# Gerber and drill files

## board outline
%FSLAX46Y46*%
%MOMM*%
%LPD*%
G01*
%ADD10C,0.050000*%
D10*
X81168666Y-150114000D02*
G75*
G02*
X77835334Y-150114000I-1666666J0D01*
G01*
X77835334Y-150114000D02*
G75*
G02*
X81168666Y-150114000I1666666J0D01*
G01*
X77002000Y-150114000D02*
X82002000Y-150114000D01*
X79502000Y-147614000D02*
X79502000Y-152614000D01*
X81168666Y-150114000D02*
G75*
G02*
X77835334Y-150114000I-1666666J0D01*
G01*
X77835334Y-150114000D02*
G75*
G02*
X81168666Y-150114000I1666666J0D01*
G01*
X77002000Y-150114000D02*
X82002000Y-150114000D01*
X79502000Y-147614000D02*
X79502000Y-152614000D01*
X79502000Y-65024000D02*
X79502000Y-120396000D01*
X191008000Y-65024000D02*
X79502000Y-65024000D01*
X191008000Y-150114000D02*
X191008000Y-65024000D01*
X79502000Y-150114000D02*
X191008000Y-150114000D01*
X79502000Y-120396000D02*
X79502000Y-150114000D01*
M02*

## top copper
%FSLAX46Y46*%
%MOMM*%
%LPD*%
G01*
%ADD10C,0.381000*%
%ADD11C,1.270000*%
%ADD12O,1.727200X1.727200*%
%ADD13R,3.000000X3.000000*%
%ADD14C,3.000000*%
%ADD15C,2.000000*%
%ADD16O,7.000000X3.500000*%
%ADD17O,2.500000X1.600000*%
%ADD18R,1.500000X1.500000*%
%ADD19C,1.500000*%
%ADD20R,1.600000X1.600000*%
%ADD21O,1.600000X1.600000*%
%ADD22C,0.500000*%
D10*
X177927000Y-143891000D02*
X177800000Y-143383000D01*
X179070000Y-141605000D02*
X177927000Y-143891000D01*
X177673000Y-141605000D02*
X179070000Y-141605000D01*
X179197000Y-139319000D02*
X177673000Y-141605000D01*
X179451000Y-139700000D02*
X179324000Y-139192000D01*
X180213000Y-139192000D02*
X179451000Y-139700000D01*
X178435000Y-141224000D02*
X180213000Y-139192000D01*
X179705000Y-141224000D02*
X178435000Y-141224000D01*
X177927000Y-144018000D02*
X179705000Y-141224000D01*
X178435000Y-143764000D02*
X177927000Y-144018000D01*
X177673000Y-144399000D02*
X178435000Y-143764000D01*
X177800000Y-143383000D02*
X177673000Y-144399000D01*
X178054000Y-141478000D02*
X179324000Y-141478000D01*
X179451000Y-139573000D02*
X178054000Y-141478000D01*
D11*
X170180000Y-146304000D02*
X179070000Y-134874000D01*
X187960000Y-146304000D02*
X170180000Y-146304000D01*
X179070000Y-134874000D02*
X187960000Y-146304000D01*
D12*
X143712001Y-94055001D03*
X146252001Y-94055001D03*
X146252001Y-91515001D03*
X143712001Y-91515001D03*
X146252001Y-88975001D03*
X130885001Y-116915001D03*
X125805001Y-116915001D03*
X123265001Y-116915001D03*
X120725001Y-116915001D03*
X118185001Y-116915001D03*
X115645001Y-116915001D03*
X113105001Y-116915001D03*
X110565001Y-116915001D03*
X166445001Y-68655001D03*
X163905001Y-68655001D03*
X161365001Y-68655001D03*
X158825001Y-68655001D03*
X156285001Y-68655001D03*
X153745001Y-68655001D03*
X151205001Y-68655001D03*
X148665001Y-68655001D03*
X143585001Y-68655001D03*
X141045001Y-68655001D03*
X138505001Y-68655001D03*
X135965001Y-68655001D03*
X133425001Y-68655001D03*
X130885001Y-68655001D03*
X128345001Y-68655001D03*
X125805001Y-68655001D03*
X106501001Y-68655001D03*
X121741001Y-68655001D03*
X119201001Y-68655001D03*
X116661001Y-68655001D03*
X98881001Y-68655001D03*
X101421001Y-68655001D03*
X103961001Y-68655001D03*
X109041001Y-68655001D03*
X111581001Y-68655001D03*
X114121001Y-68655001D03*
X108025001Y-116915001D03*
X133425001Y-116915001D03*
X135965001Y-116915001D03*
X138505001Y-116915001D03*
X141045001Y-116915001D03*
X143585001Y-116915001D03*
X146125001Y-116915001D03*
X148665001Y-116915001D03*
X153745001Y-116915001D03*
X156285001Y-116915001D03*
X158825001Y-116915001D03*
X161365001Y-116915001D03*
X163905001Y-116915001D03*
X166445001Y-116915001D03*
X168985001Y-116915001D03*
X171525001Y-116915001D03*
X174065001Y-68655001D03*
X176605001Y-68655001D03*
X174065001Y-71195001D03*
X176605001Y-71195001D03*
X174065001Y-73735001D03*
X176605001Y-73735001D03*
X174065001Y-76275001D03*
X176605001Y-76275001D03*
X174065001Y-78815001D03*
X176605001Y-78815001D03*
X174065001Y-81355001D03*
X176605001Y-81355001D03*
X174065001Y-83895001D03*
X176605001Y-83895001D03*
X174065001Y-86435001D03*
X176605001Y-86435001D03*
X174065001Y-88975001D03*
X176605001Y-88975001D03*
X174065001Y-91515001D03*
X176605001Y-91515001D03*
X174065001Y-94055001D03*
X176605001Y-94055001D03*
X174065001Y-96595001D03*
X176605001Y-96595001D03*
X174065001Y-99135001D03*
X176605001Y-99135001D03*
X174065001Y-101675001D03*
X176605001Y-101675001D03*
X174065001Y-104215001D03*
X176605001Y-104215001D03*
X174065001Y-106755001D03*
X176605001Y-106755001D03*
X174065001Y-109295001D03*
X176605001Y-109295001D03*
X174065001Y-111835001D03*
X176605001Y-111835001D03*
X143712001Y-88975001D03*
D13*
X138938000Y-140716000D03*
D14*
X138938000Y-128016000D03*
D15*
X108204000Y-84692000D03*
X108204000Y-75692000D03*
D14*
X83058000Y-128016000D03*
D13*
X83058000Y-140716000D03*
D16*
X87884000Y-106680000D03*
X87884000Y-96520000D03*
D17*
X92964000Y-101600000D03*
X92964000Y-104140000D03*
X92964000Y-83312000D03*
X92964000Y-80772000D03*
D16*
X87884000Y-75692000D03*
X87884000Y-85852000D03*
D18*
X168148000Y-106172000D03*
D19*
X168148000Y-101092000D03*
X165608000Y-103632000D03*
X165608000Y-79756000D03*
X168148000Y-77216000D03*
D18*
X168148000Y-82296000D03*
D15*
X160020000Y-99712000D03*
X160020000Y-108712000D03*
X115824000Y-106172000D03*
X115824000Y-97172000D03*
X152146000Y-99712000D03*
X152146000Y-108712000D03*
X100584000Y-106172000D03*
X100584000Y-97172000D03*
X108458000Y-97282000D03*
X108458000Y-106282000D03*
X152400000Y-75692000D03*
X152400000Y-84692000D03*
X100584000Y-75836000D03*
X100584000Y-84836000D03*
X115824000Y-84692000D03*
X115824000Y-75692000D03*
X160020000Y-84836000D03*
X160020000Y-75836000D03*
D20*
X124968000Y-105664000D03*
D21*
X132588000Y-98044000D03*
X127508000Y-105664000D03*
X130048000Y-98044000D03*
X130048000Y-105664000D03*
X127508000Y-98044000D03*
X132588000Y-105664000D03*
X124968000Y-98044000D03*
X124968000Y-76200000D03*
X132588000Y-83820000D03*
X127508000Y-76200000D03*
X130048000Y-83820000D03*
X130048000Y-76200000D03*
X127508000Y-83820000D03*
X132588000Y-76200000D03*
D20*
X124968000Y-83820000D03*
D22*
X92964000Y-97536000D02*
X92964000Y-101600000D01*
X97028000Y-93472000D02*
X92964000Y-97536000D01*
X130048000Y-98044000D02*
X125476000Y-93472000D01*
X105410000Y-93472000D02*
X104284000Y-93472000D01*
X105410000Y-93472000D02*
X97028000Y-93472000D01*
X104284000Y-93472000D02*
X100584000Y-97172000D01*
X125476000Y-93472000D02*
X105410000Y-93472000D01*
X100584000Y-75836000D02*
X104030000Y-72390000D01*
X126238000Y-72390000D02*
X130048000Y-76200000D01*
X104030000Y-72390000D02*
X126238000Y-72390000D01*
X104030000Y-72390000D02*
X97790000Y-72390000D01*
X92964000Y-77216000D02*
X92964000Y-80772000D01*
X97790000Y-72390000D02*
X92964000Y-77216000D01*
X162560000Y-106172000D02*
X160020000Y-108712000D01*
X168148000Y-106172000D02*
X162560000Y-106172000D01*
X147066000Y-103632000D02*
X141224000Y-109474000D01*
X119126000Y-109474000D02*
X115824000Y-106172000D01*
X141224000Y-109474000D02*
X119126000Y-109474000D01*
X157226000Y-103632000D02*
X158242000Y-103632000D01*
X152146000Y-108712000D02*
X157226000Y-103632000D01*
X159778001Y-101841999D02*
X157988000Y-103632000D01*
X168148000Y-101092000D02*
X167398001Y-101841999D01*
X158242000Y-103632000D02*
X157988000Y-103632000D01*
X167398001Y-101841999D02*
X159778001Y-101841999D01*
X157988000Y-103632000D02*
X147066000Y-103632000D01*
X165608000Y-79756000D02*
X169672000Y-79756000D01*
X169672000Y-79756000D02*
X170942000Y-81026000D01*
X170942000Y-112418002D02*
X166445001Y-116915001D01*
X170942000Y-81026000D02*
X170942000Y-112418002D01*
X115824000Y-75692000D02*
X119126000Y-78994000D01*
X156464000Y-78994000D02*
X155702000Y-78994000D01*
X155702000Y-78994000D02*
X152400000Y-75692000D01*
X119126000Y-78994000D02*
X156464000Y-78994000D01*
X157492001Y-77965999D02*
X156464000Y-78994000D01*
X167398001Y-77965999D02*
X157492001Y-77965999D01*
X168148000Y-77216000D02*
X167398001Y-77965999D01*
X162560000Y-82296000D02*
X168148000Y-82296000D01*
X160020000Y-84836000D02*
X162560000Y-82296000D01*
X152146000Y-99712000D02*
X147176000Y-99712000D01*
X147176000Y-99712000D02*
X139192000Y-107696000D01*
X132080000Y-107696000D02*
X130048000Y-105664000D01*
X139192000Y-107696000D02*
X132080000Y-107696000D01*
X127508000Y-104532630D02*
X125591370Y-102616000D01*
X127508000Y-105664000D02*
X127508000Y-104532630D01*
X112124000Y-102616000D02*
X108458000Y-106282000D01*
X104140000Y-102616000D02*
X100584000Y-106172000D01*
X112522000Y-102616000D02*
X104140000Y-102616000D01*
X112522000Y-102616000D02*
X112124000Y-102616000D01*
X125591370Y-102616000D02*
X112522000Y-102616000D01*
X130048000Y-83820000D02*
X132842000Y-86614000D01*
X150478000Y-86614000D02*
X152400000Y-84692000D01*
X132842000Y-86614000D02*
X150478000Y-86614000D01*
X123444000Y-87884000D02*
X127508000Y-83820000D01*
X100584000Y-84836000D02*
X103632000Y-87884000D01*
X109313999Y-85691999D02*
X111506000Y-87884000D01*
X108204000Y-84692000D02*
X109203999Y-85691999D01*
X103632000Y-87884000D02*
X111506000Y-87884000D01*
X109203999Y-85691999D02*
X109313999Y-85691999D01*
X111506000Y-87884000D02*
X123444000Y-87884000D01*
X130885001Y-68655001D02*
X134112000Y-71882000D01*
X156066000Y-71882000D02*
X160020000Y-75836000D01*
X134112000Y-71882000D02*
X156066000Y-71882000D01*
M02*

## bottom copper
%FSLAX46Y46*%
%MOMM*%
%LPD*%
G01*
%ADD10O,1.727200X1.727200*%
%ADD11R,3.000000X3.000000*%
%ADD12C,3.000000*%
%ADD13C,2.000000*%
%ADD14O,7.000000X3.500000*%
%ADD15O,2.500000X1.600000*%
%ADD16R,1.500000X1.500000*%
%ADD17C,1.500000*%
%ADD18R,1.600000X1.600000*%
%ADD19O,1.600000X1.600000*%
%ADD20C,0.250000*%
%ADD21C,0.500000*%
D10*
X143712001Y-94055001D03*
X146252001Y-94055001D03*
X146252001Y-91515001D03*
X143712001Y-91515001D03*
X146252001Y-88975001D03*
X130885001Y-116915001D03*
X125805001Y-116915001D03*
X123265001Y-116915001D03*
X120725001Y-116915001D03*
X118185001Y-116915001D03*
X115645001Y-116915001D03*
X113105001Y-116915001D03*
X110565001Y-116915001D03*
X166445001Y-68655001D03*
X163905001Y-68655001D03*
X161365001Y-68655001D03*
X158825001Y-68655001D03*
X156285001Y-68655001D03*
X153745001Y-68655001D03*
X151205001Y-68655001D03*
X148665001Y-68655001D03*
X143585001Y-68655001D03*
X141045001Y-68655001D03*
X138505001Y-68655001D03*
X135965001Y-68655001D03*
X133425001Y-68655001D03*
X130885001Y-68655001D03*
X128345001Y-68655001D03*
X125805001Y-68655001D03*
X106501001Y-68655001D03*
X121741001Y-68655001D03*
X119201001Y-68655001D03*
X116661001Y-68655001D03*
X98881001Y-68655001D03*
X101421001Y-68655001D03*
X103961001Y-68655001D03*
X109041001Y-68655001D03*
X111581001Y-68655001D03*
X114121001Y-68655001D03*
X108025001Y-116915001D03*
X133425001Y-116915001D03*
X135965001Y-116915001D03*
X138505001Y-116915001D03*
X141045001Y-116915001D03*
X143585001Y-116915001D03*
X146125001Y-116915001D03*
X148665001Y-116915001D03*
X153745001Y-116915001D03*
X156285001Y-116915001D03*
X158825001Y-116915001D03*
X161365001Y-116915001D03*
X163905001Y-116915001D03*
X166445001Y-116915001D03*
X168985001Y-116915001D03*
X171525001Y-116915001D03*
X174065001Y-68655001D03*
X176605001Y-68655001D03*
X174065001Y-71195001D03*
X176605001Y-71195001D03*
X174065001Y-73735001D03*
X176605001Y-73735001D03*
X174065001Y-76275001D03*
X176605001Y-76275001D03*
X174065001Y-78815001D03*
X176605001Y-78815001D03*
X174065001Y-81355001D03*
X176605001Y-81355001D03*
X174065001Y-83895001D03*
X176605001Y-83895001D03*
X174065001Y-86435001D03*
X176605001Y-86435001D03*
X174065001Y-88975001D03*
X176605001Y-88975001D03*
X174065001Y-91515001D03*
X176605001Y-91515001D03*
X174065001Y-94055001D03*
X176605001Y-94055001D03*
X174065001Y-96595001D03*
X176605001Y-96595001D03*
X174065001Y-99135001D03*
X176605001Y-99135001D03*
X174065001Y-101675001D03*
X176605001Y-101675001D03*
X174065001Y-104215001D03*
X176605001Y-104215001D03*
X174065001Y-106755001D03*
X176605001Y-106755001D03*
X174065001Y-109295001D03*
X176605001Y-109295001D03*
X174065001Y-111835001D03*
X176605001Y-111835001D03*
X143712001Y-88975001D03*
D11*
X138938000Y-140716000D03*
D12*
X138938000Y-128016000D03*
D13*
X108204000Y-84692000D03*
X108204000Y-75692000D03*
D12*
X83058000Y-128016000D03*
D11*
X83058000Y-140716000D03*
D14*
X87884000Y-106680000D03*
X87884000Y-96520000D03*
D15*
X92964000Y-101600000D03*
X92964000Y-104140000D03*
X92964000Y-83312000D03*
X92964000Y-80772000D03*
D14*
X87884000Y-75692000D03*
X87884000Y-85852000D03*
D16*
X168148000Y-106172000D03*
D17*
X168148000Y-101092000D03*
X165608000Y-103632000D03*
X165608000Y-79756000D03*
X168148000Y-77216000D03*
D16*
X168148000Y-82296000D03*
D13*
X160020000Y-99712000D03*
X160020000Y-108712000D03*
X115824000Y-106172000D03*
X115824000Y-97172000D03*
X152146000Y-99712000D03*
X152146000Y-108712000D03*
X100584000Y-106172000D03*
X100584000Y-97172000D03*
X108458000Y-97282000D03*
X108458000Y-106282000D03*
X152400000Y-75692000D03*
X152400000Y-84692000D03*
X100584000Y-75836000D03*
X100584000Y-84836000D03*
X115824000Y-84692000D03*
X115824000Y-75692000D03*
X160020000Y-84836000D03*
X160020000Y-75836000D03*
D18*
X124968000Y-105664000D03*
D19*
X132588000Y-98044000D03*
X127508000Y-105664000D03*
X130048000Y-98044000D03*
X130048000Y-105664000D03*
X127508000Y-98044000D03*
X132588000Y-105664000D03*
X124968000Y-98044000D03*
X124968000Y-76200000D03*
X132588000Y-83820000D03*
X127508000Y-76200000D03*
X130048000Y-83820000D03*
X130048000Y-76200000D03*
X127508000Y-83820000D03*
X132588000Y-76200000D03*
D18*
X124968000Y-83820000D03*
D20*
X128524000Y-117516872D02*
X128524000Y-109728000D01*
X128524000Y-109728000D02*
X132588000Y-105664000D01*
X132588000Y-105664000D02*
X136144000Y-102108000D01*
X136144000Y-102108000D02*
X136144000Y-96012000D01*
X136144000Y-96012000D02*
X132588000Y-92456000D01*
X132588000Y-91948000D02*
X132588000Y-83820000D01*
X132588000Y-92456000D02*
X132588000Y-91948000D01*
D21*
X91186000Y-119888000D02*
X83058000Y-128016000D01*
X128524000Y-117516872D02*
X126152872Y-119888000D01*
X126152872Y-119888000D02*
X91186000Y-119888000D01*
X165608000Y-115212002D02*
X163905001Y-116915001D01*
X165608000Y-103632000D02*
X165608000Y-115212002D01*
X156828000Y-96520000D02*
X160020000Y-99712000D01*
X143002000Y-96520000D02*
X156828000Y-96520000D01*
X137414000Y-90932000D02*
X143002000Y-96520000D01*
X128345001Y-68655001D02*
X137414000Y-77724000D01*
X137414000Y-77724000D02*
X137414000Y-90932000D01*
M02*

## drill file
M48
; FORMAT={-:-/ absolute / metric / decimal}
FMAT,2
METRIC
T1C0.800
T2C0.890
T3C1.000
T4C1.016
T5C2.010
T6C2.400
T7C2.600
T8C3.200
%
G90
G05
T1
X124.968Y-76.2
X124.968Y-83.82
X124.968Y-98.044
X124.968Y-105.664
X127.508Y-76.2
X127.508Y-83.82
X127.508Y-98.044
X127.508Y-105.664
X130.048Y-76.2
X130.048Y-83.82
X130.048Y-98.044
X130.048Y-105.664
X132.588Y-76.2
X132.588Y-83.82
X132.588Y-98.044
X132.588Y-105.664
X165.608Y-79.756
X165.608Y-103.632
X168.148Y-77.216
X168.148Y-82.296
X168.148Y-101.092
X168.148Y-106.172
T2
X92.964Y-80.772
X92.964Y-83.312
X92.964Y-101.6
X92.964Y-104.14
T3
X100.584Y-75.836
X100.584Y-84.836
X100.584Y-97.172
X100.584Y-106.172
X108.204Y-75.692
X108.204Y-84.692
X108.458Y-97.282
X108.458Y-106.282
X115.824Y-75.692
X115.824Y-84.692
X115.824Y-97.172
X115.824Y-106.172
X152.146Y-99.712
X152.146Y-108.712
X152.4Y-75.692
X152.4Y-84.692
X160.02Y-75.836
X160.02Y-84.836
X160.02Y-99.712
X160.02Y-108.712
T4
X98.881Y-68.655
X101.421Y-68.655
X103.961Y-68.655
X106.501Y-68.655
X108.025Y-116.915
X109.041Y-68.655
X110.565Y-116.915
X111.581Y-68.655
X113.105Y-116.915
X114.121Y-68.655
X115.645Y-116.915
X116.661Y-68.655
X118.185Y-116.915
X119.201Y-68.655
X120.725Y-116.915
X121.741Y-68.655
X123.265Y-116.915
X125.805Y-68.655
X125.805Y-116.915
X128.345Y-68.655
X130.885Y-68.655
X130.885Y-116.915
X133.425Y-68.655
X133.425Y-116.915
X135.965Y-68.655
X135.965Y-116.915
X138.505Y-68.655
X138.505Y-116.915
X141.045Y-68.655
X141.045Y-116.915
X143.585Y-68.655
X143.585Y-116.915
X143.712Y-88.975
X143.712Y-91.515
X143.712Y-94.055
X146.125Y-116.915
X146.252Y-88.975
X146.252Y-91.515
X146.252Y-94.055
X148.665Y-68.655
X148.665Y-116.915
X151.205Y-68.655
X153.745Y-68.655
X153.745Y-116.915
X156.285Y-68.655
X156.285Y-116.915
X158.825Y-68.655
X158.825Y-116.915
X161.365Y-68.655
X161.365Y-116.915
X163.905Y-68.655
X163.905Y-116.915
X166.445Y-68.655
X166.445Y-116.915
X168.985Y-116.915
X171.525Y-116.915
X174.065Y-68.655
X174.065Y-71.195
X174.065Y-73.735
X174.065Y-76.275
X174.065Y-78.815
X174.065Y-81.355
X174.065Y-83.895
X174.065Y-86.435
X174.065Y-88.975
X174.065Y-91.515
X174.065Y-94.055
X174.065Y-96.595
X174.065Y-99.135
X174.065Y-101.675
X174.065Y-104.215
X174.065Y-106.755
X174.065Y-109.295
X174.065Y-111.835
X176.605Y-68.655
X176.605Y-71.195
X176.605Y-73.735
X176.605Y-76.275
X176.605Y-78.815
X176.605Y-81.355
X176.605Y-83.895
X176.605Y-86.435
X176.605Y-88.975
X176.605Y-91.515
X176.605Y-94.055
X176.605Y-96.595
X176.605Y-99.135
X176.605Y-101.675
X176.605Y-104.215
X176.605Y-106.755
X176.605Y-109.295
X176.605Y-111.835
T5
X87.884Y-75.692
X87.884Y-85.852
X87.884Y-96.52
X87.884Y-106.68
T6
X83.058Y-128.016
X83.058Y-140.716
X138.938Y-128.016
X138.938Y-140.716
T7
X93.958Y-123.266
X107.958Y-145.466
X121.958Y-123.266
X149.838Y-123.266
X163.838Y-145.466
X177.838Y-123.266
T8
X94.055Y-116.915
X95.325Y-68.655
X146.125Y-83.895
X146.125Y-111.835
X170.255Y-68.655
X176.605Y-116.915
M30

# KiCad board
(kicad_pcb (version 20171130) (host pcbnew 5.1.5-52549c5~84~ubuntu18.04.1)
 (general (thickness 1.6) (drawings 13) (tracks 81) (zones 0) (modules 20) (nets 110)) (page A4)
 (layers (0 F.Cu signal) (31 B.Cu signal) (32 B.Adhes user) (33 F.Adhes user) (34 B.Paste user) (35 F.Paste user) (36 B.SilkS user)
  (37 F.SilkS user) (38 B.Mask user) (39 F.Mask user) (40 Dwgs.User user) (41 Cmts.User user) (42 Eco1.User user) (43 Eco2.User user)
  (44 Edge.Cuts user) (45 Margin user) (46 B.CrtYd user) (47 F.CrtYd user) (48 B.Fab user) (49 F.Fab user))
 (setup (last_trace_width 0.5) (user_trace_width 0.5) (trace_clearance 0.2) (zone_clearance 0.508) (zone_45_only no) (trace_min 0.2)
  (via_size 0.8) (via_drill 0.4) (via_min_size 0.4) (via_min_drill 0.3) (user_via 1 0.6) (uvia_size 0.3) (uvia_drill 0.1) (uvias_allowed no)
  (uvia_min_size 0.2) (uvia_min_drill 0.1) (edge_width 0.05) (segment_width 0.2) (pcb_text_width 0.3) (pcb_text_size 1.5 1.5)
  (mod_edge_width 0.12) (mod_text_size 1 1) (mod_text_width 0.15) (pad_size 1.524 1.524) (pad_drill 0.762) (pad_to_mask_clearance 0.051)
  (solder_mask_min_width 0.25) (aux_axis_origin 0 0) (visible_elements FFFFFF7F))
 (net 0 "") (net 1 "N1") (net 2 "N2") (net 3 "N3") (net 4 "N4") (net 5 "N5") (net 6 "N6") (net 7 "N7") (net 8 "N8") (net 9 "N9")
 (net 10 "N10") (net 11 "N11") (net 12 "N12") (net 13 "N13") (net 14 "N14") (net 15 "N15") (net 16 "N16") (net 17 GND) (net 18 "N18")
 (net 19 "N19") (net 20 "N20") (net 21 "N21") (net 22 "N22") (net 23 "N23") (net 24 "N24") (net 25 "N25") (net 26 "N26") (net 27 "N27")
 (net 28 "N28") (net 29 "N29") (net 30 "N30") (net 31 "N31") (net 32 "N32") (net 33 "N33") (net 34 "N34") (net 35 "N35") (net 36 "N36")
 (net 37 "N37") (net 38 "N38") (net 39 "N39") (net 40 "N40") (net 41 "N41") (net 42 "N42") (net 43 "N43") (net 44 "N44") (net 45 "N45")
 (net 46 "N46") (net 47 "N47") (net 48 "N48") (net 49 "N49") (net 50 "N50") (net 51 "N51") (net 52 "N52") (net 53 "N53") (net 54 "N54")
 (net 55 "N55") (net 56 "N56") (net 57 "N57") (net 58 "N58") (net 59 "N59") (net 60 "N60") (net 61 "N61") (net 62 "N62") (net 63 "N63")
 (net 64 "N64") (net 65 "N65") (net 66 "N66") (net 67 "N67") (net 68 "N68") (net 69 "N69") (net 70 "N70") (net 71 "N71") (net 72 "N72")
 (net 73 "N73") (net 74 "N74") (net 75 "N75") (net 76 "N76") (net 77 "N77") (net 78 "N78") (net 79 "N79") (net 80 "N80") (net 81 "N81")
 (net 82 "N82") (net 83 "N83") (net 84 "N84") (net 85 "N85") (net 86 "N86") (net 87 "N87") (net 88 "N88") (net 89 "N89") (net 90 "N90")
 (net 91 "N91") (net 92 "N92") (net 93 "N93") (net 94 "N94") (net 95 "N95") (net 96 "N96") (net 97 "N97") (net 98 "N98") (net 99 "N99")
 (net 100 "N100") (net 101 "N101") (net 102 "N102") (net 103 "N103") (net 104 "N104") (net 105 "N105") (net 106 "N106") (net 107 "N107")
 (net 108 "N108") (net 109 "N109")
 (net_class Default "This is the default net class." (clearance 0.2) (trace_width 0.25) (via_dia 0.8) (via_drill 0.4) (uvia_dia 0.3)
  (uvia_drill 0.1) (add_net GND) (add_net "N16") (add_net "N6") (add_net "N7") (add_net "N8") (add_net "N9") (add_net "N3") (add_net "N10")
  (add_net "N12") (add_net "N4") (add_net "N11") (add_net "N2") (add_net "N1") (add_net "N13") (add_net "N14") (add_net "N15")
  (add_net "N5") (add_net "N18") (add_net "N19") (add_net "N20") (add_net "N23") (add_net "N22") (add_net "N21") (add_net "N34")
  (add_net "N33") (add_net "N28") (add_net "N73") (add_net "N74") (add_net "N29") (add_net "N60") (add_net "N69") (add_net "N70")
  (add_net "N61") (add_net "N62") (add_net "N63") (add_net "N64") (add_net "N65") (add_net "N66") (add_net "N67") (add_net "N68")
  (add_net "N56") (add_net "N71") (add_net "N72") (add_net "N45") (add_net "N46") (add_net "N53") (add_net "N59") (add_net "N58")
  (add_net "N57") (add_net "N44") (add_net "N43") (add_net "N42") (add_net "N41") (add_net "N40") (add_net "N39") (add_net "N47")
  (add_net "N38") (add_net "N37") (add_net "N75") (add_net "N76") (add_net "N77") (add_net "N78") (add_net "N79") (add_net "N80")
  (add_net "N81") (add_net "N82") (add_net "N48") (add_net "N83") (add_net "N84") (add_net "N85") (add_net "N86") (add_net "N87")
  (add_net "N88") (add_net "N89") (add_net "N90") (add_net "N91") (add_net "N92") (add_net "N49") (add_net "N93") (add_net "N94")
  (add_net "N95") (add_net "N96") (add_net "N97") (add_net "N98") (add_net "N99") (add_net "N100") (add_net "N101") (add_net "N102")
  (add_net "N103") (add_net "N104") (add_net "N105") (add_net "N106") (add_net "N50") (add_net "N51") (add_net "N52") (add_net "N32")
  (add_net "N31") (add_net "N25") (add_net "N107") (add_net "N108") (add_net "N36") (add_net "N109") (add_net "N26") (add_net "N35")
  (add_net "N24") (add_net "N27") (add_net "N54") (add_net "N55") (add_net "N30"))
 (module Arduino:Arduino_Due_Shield (layer F.Cu) (at 80.085001 119.455001)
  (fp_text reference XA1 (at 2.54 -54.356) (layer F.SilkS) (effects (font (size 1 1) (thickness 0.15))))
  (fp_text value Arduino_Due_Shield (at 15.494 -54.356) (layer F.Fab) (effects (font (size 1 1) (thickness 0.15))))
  (pad RST2 thru_hole oval (at 63.627 -25.4) (size 1.7272 1.7272) (drill 1.016) (layers *.Cu *.Mask))
  (pad GND4 thru_hole oval (at 66.167 -25.4) (size 1.7272 1.7272) (drill 1.016) (layers *.Cu *.Mask))
  (pad MOSI thru_hole oval (at 66.167 -27.94) (size 1.7272 1.7272) (drill 1.016) (layers *.Cu *.Mask))
  (pad SCK thru_hole oval (at 63.627 -27.94) (size 1.7272 1.7272) (drill 1.016) (layers *.Cu *.Mask))
  (pad 5V2 thru_hole oval (at 66.167 -30.48) (size 1.7272 1.7272) (drill 1.016) (layers *.Cu *.Mask))
  (pad A0 thru_hole oval (at 50.8 -2.54) (size 1.7272 1.7272) (drill 1.016) (layers *.Cu *.Mask))
  (pad VIN thru_hole oval (at 45.72 -2.54) (size 1.7272 1.7272) (drill 1.016) (layers *.Cu *.Mask))
  (pad GND3 thru_hole oval (at 43.18 -2.54) (size 1.7272 1.7272) (drill 1.016) (layers *.Cu *.Mask))
  (pad GND2 thru_hole oval (at 40.64 -2.54) (size 1.7272 1.7272) (drill 1.016) (layers *.Cu *.Mask))
  (pad 5V1 thru_hole oval (at 38.1 -2.54) (size 1.7272 1.7272) (drill 1.016) (layers *.Cu *.Mask))
  (pad 3V3 thru_hole oval (at 35.56 -2.54) (size 1.7272 1.7272) (drill 1.016) (layers *.Cu *.Mask))
  (pad RST1 thru_hole oval (at 33.02 -2.54) (size 1.7272 1.7272) (drill 1.016) (layers *.Cu *.Mask))
  (pad IORF thru_hole oval (at 30.48 -2.54) (size 1.7272 1.7272) (drill 1.016) (layers *.Cu *.Mask))
  (pad D21 thru_hole oval (at 86.36 -50.8) (size 1.7272 1.7272) (drill 1.016) (layers *.Cu *.Mask))
  (pad D20 thru_hole oval (at 83.82 -50.8) (size 1.7272 1.7272) (drill 1.016) (layers *.Cu *.Mask))
  (pad D19 thru_hole oval (at 81.28 -50.8) (size 1.7272 1.7272) (drill 1.016) (layers *.Cu *.Mask))
  (pad D18 thru_hole oval (at 78.74 -50.8) (size 1.7272 1.7272) (drill 1.016) (layers *.Cu *.Mask))
  (pad D17 thru_hole oval (at 76.2 -50.8) (size 1.7272 1.7272) (drill 1.016) (layers *.Cu *.Mask))
  (pad D16 thru_hole oval (at 73.66 -50.8) (size 1.7272 1.7272) (drill 1.016) (layers *.Cu *.Mask))
  (pad D15 thru_hole oval (at 71.12 -50.8) (size 1.7272 1.7272) (drill 1.016) (layers *.Cu *.Mask))
  (pad D14 thru_hole oval (at 68.58 -50.8) (size 1.7272 1.7272) (drill 1.016) (layers *.Cu *.Mask))
  (pad D0 thru_hole oval (at 63.5 -50.8) (size 1.7272 1.7272) (drill 1.016) (layers *.Cu *.Mask))
  (pad D1 thru_hole oval (at 60.96 -50.8) (size 1.7272 1.7272) (drill 1.016) (layers *.Cu *.Mask))
  (pad D2 thru_hole oval (at 58.42 -50.8) (size 1.7272 1.7272) (drill 1.016) (layers *.Cu *.Mask))
  (pad D3 thru_hole oval (at 55.88 -50.8) (size 1.7272 1.7272) (drill 1.016) (layers *.Cu *.Mask))
  (pad D4 thru_hole oval (at 53.34 -50.8) (size 1.7272 1.7272) (drill 1.016) (layers *.Cu *.Mask))
  (pad D5 thru_hole oval (at 50.8 -50.8) (size 1.7272 1.7272) (drill 1.016) (layers *.Cu *.Mask) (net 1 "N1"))
  (pad D6 thru_hole oval (at 48.26 -50.8) (size 1.7272 1.7272) (drill 1.016) (layers *.Cu *.Mask) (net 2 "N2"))
  (pad D7 thru_hole oval (at 45.72 -50.8) (size 1.7272 1.7272) (drill 1.016) (layers *.Cu *.Mask))
  (pad GND1 thru_hole oval (at 26.416 -50.8) (size 1.7272 1.7272) (drill 1.016) (layers *.Cu *.Mask))
  (pad D8 thru_hole oval (at 41.656 -50.8) (size 1.7272 1.7272) (drill 1.016) (layers *.Cu *.Mask))
  (pad D9 thru_hole oval (at 39.116 -50.8) (size 1.7272 1.7272) (drill 1.016) (layers *.Cu *.Mask))
  (pad D10 thru_hole oval (at 36.576 -50.8) (size 1.7272 1.7272) (drill 1.016) (layers *.Cu *.Mask))
  (pad "" np_thru_hole circle (at 66.04 -7.62) (size 3.2 3.2) (drill 3.2) (layers *.Cu *.Mask))
  (pad "" np_thru_hole circle (at 66.04 -35.56) (size 3.2 3.2) (drill 3.2) (layers *.Cu *.Mask))
  (pad "" np_thru_hole circle (at 90.17 -50.8) (size 3.2 3.2) (drill 3.2) (layers *.Cu *.Mask))
  (pad "" np_thru_hole circle (at 15.24 -50.8) (size 3.2 3.2) (drill 3.2) (layers *.Cu *.Mask))
  (pad "" np_thru_hole circle (at 96.52 -2.54) (size 3.2 3.2) (drill 3.2) (layers *.Cu *.Mask))
  (pad "" np_thru_hole circle (at 13.97 -2.54) (size 3.2 3.2) (drill 3.2) (layers *.Cu *.Mask))
  (pad SCL1 thru_hole oval (at 18.796 -50.8) (size 1.7272 1.7272) (drill 1.016) (layers *.Cu *.Mask))
  (pad SDA1 thru_hole oval (at 21.336 -50.8) (size 1.7272 1.7272) (drill 1.016) (layers *.Cu *.Mask))
  (pad AREF thru_hole oval (at 23.876 -50.8) (size 1.7272 1.7272) (drill 1.016) (layers *.Cu *.Mask))
  (pad D13 thru_hole oval (at 28.956 -50.8) (size 1.7272 1.7272) (drill 1.016) (layers *.Cu *.Mask))
  (pad D12 thru_hole oval (at 31.496 -50.8) (size 1.7272 1.7272) (drill 1.016) (layers *.Cu *.Mask))
  (pad D11 thru_hole oval (at 34.036 -50.8) (size 1.7272 1.7272) (drill 1.016) (layers *.Cu *.Mask))
  (pad "" thru_hole oval (at 27.94 -2.54) (size 1.7272 1.7272) (drill 1.016) (layers *.Cu *.Mask))
  (pad A1 thru_hole oval (at 53.34 -2.54) (size 1.7272 1.7272) (drill 1.016) (layers *.Cu *.Mask))
  (pad A2 thru_hole oval (at 55.88 -2.54) (size 1.7272 1.7272) (drill 1.016) (layers *.Cu *.Mask))
  (pad A3 thru_hole oval (at 58.42 -2.54) (size 1.7272 1.7272) (drill 1.016) (layers *.Cu *.Mask))
  (pad A4 thru_hole oval (at 60.96 -2.54) (size 1.7272 1.7272) (drill 1.016) (layers *.Cu *.Mask))
  (pad A5 thru_hole oval (at 63.5 -2.54) (size 1.7272 1.7272) (drill 1.016) (layers *.Cu *.Mask))
  (pad A6 thru_hole oval (at 66.04 -2.54) (size 1.7272 1.7272) (drill 1.016) (layers *.Cu *.Mask))
  (pad A7 thru_hole oval (at 68.58 -2.54) (size 1.7272 1.7272) (drill 1.016) (layers *.Cu *.Mask))
  (pad A8 thru_hole oval (at 73.66 -2.54) (size 1.7272 1.7272) (drill 1.016) (layers *.Cu *.Mask))
  (pad A9 thru_hole oval (at 76.2 -2.54) (size 1.7272 1.7272) (drill 1.016) (layers *.Cu *.Mask))
  (pad A10 thru_hole oval (at 78.74 -2.54) (size 1.7272 1.7272) (drill 1.016) (layers *.Cu *.Mask))
  (pad A11 thru_hole oval (at 81.28 -2.54) (size 1.7272 1.7272) (drill 1.016) (layers *.Cu *.Mask))
  (pad DAC0 thru_hole oval (at 83.82 -2.54) (size 1.7272 1.7272) (drill 1.016) (layers *.Cu *.Mask) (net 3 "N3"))
  (pad DAC1 thru_hole oval (at 86.36 -2.54) (size 1.7272 1.7272) (drill 1.016) (layers *.Cu *.Mask) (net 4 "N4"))
  (pad CANR thru_hole oval (at 88.9 -2.54) (size 1.7272 1.7272) (drill 1.016) (layers *.Cu *.Mask))
  (pad CANT thru_hole oval (at 91.44 -2.54) (size 1.7272 1.7272) (drill 1.016) (layers *.Cu *.Mask))
  (pad 5V3 thru_hole oval (at 93.98 -50.8) (size 1.7272 1.7272) (drill 1.016) (layers *.Cu *.Mask))
  (pad 5V4 thru_hole oval (at 96.52 -50.8) (size 1.7272 1.7272) (drill 1.016) (layers *.Cu *.Mask))
  (pad D22 thru_hole oval (at 93.98 -48.26) (size 1.7272 1.7272) (drill 1.016) (layers *.Cu *.Mask))
  (pad D23 thru_hole oval (at 96.52 -48.26) (size 1.7272 1.7272) (drill 1.016) (layers *.Cu *.Mask))
  (pad D24 thru_hole oval (at 93.98 -45.72) (size 1.7272 1.7272) (drill 1.016) (layers *.Cu *.Mask))
  (pad D25 thru_hole oval (at 96.52 -45.72) (size 1.7272 1.7272) (drill 1.016) (layers *.Cu *.Mask))
  (pad D26 thru_hole oval (at 93.98 -43.18) (size 1.7272 1.7272) (drill 1.016) (layers *.Cu *.Mask))
  (pad D27 thru_hole oval (at 96.52 -43.18) (size 1.7272 1.7272) (drill 1.016) (layers *.Cu *.Mask))
  (pad D28 thru_hole oval (at 93.98 -40.64) (size 1.7272 1.7272) (drill 1.016) (layers *.Cu *.Mask))
  (pad D29 thru_hole oval (at 96.52 -40.64) (size 1.7272 1.7272) (drill 1.016) (layers *.Cu *.Mask))
  (pad D30 thru_hole oval (at 93.98 -38.1) (size 1.7272 1.7272) (drill 1.016) (layers *.Cu *.Mask))
  (pad D31 thru_hole oval (at 96.52 -38.1) (size 1.7272 1.7272) (drill 1.016) (layers *.Cu *.Mask))
  (pad D32 thru_hole oval (at 93.98 -35.56) (size 1.7272 1.7272) (drill 1.016) (layers *.Cu *.Mask))
  (pad D33 thru_hole oval (at 96.52 -35.56) (size 1.7272 1.7272) (drill 1.016) (layers *.Cu *.Mask))
  (pad D34 thru_hole oval (at 93.98 -33.02) (size 1.7272 1.7272) (drill 1.016) (layers *.Cu *.Mask))
  (pad D35 thru_hole oval (at 96.52 -33.02) (size 1.7272 1.7272) (drill 1.016) (layers *.Cu *.Mask))
  (pad D36 thru_hole oval (at 93.98 -30.48) (size 1.7272 1.7272) (drill 1.016) (layers *.Cu *.Mask))
  (pad D37 thru_hole oval (at 96.52 -30.48) (size 1.7272 1.7272) (drill 1.016) (layers *.Cu *.Mask))
  (pad D38 thru_hole oval (at 93.98 -27.94) (size 1.7272 1.7272) (drill 1.016) (layers *.Cu *.Mask))
  (pad D39 thru_hole oval (at 96.52 -27.94) (size 1.7272 1.7272) (drill 1.016) (layers *.Cu *.Mask))
  (pad D40 thru_hole oval (at 93.98 -25.4) (size 1.7272 1.7272) (drill 1.016) (layers *.Cu *.Mask))
  (pad D41 thru_hole oval (at 96.52 -25.4) (size 1.7272 1.7272) (drill 1.016) (layers *.Cu *.Mask))
  (pad D42 thru_hole oval (at 93.98 -22.86) (size 1.7272 1.7272) (drill 1.016) (layers *.Cu *.Mask))
  (pad D43 thru_hole oval (at 96.52 -22.86) (size 1.7272 1.7272) (drill 1.016) (layers *.Cu *.Mask))
  (pad D44 thru_hole oval (at 93.98 -20.32) (size 1.7272 1.7272) (drill 1.016) (layers *.Cu *.Mask))
  (pad D45 thru_hole oval (at 96.52 -20.32) (size 1.7272 1.7272) (drill 1.016) (layers *.Cu *.Mask))
  (pad D46 thru_hole oval (at 93.98 -17.78) (size 1.7272 1.7272) (drill 1.016) (layers *.Cu *.Mask))
  (pad D47 thru_hole oval (at 96.52 -17.78) (size 1.7272 1.7272) (drill 1.016) (layers *.Cu *.Mask))
  (pad D48 thru_hole oval (at 93.98 -15.24) (size 1.7272 1.7272) (drill 1.016) (layers *.Cu *.Mask))
  (pad D49 thru_hole oval (at 96.52 -15.24) (size 1.7272 1.7272) (drill 1.016) (layers *.Cu *.Mask))
  (pad D50 thru_hole oval (at 93.98 -12.7) (size 1.7272 1.7272) (drill 1.016) (layers *.Cu *.Mask))
  (pad D51 thru_hole oval (at 96.52 -12.7) (size 1.7272 1.7272) (drill 1.016) (layers *.Cu *.Mask))
  (pad D52 thru_hole oval (at 93.98 -10.16) (size 1.7272 1.7272) (drill 1.016) (layers *.Cu *.Mask))
  (pad D53 thru_hole oval (at 96.52 -10.16) (size 1.7272 1.7272) (drill 1.016) (layers *.Cu *.Mask))
  (pad GND5 thru_hole oval (at 93.98 -7.62) (size 1.7272 1.7272) (drill 1.016) (layers *.Cu *.Mask))
  (pad GND6 thru_hole oval (at 96.52 -7.62) (size 1.7272 1.7272) (drill 1.016) (layers *.Cu *.Mask))
  (pad MISO thru_hole oval (at 63.627 -30.48) (size 1.7272 1.7272) (drill 1.016) (layers *.Cu *.Mask)))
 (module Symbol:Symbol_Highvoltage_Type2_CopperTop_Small (layer F.Cu) (at 179.07 142.494)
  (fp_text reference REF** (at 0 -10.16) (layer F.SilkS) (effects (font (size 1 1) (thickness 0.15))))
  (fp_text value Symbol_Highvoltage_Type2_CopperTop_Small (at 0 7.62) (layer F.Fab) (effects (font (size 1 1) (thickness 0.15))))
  (fp_line (start -1.143 1.397) (end -1.27 0.889) (layer F.Cu) (width 0.381))
  (fp_line (start 0 -0.889) (end -1.143 1.397) (layer F.Cu) (width 0.381))
  (fp_line (start -1.397 -0.889) (end 0 -0.889) (layer F.Cu) (width 0.381))
  (fp_line (start 0.127 -3.175) (end -1.397 -0.889) (layer F.Cu) (width 0.381))
  (fp_line (start 0.381 -2.794) (end 0.254 -3.302) (layer F.Cu) (width 0.381))
  (fp_line (start 1.143 -3.302) (end 0.381 -2.794) (layer F.Cu) (width 0.381))
  (fp_line (start -0.635 -1.27) (end 1.143 -3.302) (layer F.Cu) (width 0.381))
  (fp_line (start 0.635 -1.27) (end -0.635 -1.27) (layer F.Cu) (width 0.381))
  (fp_line (start -1.143 1.524) (end 0.635 -1.27) (layer F.Cu) (width 0.381))
  (fp_line (start -0.635 1.27) (end -1.143 1.524) (layer F.Cu) (width 0.381))
  (fp_line (start -1.397 1.905) (end -0.635 1.27) (layer F.Cu) (width 0.381))
  (fp_line (start -1.27 0.889) (end -1.397 1.905) (layer F.Cu) (width 0.381))
  (fp_line (start -1.016 -1.016) (end 0.254 -1.016) (layer F.Cu) (width 0.381))
  (fp_line (start 0.381 -2.921) (end -1.016 -1.016) (layer F.Cu) (width 0.381))
  (fp_line (start -8.89 3.81) (end 0 -7.62) (layer F.Cu) (width 1.27))
  (fp_line (start 8.89 3.81) (end -8.89 3.81) (layer F.Cu) (width 1.27))
  (fp_line (start 0 -7.62) (end 8.89 3.81) (layer F.Cu) (width 1.27)))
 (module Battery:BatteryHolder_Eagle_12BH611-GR (layer B.Cu) (at 138.938 140.716 180)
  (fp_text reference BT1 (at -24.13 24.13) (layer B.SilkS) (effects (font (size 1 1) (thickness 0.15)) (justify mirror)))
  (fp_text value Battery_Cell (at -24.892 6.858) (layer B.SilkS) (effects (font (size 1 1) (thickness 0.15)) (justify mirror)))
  (pad "" np_thru_hole circle (at -24.9 -4.75 180) (size 2.6 2.6) (drill 2.6) (layers *.Cu *.Mask))
  (pad "" np_thru_hole circle (at -38.9 17.45 180) (size 2.6 2.6) (drill 2.6) (layers *.Cu *.Mask))
  (pad "" np_thru_hole circle (at -10.9 17.45 180) (size 2.6 2.6) (drill 2.6) (layers *.Cu *.Mask))
  (pad 1 thru_hole rect (at 0 0 180) (size 3 3) (drill 2.4) (layers *.Cu *.Mask))
  (pad 2 thru_hole circle (at 0 12.7 180) (size 3 3) (drill 2.4) (layers *.Cu *.Mask)))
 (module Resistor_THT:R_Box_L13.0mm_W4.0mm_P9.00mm (layer F.Cu) (at 108.204 75.692 270)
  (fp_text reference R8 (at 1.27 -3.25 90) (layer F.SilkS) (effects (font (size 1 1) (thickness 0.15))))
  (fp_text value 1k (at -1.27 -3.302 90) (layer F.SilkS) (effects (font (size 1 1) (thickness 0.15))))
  (pad 2 thru_hole circle (at 9 0 270) (size 2 2) (drill 1) (layers *.Cu *.Mask) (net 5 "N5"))
  (pad 1 thru_hole circle (at 0 0 270) (size 2 2) (drill 1) (layers *.Cu *.Mask)))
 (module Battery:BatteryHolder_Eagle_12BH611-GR (layer B.Cu) (at 83.058 140.716 180)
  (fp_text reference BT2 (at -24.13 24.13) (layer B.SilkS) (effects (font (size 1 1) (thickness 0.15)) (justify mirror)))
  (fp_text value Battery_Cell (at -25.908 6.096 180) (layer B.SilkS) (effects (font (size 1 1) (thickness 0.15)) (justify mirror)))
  (pad 2 thru_hole circle (at 0 12.7 180) (size 3 3) (drill 2.4) (layers *.Cu *.Mask) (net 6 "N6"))
  (pad 1 thru_hole rect (at 0 0 180) (size 3 3) (drill 2.4) (layers *.Cu *.Mask))
  (pad "" np_thru_hole circle (at -10.9 17.45 180) (size 2.6 2.6) (drill 2.6) (layers *.Cu *.Mask))
  (pad "" np_thru_hole circle (at -38.9 17.45 180) (size 2.6 2.6) (drill 2.6) (layers *.Cu *.Mask))
  (pad "" np_thru_hole circle (at -24.9 -4.75 180) (size 2.6 2.6) (drill 2.6) (layers *.Cu *.Mask)))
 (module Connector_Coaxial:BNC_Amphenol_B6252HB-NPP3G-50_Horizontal (layer F.Cu) (at 92.964 101.6 90)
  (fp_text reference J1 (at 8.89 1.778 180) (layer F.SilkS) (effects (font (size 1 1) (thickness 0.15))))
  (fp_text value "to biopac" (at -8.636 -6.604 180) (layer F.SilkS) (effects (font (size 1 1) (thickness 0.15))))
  (pad 2 thru_hole oval (at -5.08 -5.08 90) (size 3.5 7) (drill 2.01) (layers *.Cu *.Mask))
  (pad 2 thru_hole oval (at 5.08 -5.08 90) (size 3.5 7) (drill 2.01) (layers *.Cu *.Mask))
  (pad 1 thru_hole oval (at 0 0 90) (size 1.6 2.5) (drill 0.89) (layers *.Cu *.Mask) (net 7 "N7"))
  (pad 2 thru_hole oval (at -2.54 0 90) (size 1.6 2.5) (drill 0.89) (layers *.Cu *.Mask)))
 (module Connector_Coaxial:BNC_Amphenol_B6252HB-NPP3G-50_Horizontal (layer F.Cu) (at 92.964 80.772 90)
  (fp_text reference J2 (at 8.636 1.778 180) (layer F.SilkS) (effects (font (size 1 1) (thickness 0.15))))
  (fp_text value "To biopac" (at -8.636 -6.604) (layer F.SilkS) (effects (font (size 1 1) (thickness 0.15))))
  (pad 2 thru_hole oval (at -2.54 0 90) (size 1.6 2.5) (drill 0.89) (layers *.Cu *.Mask))
  (pad 1 thru_hole oval (at 0 0 90) (size 1.6 2.5) (drill 0.89) (layers *.Cu *.Mask) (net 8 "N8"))
  (pad 2 thru_hole oval (at 5.08 -5.08 90) (size 3.5 7) (drill 2.01) (layers *.Cu *.Mask))
  (pad 2 thru_hole oval (at -5.08 -5.08 90) (size 3.5 7) (drill 2.01) (layers *.Cu *.Mask)))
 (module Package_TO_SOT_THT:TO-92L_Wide (layer F.Cu) (at 168.148 106.172 90)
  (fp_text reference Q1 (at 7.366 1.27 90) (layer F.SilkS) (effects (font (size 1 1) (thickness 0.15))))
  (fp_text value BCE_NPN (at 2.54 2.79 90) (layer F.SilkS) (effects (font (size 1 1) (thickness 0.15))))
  (pad 1 thru_hole rect (at 0 0 180) (size 1.5 1.5) (drill 0.8) (layers *.Cu *.Mask) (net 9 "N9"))
  (pad 3 thru_hole circle (at 5.08 0 180) (size 1.5 1.5) (drill 0.8) (layers *.Cu *.Mask) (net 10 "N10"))
  (pad 2 thru_hole circle (at 2.54 -2.54 180) (size 1.5 1.5) (drill 0.8) (layers *.Cu *.Mask) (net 3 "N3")))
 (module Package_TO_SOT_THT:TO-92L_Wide (layer F.Cu) (at 168.148 82.296 90)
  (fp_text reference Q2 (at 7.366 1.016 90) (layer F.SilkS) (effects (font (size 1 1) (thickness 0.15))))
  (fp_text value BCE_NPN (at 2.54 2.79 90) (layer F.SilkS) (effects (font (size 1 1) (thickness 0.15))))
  (pad 2 thru_hole circle (at 2.54 -2.54 180) (size 1.5 1.5) (drill 0.8) (layers *.Cu *.Mask) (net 4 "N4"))
  (pad 3 thru_hole circle (at 5.08 0 180) (size 1.5 1.5) (drill 0.8) (layers *.Cu *.Mask) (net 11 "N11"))
  (pad 1 thru_hole rect (at 0 0 180) (size 1.5 1.5) (drill 0.8) (layers *.Cu *.Mask) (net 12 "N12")))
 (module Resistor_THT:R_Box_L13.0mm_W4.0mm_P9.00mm (layer F.Cu) (at 160.02 108.712 90)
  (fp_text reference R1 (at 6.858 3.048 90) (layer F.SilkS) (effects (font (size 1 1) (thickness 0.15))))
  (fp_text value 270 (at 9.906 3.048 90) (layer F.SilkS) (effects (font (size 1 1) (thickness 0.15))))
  (pad 2 thru_hole circle (at 9 0 90) (size 2 2) (drill 1) (layers *.Cu *.Mask) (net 2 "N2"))
  (pad 1 thru_hole circle (at 0 0 90) (size 2 2) (drill 1) (layers *.Cu *.Mask) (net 9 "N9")))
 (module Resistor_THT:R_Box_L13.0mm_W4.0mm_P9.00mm (layer F.Cu) (at 115.824 106.172 90)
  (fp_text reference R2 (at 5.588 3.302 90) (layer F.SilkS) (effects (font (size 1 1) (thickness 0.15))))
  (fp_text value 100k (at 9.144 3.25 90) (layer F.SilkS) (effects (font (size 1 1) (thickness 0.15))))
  (pad 1 thru_hole circle (at 0 0 90) (size 2 2) (drill 1) (layers *.Cu *.Mask) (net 10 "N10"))
  (pad 2 thru_hole circle (at 9 0 90) (size 2 2) (drill 1) (layers *.Cu *.Mask)))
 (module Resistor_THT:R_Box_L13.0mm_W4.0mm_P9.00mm (layer F.Cu) (at 152.146 108.712 90)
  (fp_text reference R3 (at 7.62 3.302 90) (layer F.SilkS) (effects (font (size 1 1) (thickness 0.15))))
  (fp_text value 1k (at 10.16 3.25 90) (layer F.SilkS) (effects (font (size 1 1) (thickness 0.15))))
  (pad 2 thru_hole circle (at 9 0 90) (size 2 2) (drill 1) (layers *.Cu *.Mask) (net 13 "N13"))
  (pad 1 thru_hole circle (at 0 0 90) (size 2 2) (drill 1) (layers *.Cu *.Mask) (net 10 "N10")))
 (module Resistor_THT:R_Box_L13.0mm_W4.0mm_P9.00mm (layer F.Cu) (at 100.584 106.172 90)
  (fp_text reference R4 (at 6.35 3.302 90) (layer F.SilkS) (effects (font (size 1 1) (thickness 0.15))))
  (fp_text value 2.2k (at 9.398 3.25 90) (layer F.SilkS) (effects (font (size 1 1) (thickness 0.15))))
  (pad 1 thru_hole circle (at 0 0 90) (size 2 2) (drill 1) (layers *.Cu *.Mask) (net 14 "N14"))
  (pad 2 thru_hole circle (at 9 0 90) (size 2 2) (drill 1) (layers *.Cu *.Mask) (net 7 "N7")))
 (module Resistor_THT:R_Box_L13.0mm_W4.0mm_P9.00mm (layer F.Cu) (at 108.458 97.282 270)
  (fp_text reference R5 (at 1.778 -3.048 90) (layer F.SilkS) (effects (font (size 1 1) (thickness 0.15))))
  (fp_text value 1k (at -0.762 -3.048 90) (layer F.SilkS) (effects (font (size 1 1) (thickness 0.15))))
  (pad 1 thru_hole circle (at 0 0 270) (size 2 2) (drill 1) (layers *.Cu *.Mask))
  (pad 2 thru_hole circle (at 9 0 270) (size 2 2) (drill 1) (layers *.Cu *.Mask) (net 14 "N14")))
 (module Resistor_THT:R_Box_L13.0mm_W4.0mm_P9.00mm (layer F.Cu) (at 152.4 75.692 270)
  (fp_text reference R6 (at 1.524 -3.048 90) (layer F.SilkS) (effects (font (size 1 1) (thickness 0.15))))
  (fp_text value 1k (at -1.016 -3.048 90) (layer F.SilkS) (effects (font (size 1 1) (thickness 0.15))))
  (pad 1 thru_hole circle (at 0 0 270) (size 2 2) (drill 1) (layers *.Cu *.Mask) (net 11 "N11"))
  (pad 2 thru_hole circle (at 9 0 270) (size 2 2) (drill 1) (layers *.Cu *.Mask) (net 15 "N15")))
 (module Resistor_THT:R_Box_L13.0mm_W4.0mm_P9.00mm (layer F.Cu) (at 100.584 84.836 90)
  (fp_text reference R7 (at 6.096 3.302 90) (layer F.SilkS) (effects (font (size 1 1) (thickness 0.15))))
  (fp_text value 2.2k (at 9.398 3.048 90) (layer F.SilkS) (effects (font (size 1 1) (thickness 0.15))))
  (pad 2 thru_hole circle (at 9 0 90) (size 2 2) (drill 1) (layers *.Cu *.Mask) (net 8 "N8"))
  (pad 1 thru_hole circle (at 0 0 90) (size 2 2) (drill 1) (layers *.Cu *.Mask) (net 5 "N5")))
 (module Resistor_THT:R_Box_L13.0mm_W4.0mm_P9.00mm (layer F.Cu) (at 115.824 75.692 270)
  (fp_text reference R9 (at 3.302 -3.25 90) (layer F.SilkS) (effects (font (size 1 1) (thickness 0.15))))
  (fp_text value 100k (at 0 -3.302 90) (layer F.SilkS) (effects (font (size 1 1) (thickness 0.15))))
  (pad 2 thru_hole circle (at 9 0 270) (size 2 2) (drill 1) (layers *.Cu *.Mask))
  (pad 1 thru_hole circle (at 0 0 270) (size 2 2) (drill 1) (layers *.Cu *.Mask) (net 11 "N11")))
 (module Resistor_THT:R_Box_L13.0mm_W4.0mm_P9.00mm (layer F.Cu) (at 160.02 84.836 90)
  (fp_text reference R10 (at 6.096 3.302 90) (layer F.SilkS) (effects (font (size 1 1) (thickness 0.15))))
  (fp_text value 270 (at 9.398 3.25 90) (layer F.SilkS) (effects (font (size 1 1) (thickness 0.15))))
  (pad 1 thru_hole circle (at 0 0 90) (size 2 2) (drill 1) (layers *.Cu *.Mask) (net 12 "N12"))
  (pad 2 thru_hole circle (at 9 0 90) (size 2 2) (drill 1) (layers *.Cu *.Mask) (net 1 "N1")))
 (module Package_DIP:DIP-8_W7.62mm (layer F.Cu) (at 124.968 105.664 90)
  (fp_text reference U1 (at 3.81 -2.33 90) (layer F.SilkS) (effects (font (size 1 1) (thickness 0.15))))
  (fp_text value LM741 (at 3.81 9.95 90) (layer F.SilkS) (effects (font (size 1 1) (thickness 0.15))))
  (pad 1 thru_hole rect (at 0 0 90) (size 1.6 1.6) (drill 0.8) (layers *.Cu *.Mask))
  (pad 5 thru_hole oval (at 7.62 7.62 90) (size 1.6 1.6) (drill 0.8) (layers *.Cu *.Mask))
  (pad 2 thru_hole oval (at 0 2.54 90) (size 1.6 1.6) (drill 0.8) (layers *.Cu *.Mask) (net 14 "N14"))
  (pad 6 thru_hole oval (at 7.62 5.08 90) (size 1.6 1.6) (drill 0.8) (layers *.Cu *.Mask) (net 7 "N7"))
  (pad 3 thru_hole oval (at 0 5.08 90) (size 1.6 1.6) (drill 0.8) (layers *.Cu *.Mask) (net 13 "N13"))
  (pad 7 thru_hole oval (at 7.62 2.54 90) (size 1.6 1.6) (drill 0.8) (layers *.Cu *.Mask))
  (pad 4 thru_hole oval (at 0 7.62 90) (size 1.6 1.6) (drill 0.8) (layers *.Cu *.Mask) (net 6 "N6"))
  (pad 8 thru_hole oval (at 7.62 0 90) (size 1.6 1.6) (drill 0.8) (layers *.Cu *.Mask)))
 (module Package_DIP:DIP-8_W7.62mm (layer F.Cu) (at 124.968 83.82 90)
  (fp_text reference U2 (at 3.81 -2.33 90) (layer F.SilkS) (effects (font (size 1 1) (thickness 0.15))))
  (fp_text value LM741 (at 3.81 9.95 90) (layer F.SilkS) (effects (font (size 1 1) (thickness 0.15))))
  (pad 8 thru_hole oval (at 7.62 0 90) (size 1.6 1.6) (drill 0.8) (layers *.Cu *.Mask))
  (pad 4 thru_hole oval (at 0 7.62 90) (size 1.6 1.6) (drill 0.8) (layers *.Cu *.Mask) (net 6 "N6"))
  (pad 7 thru_hole oval (at 7.62 2.54 90) (size 1.6 1.6) (drill 0.8) (layers *.Cu *.Mask))
  (pad 3 thru_hole oval (at 0 5.08 90) (size 1.6 1.6) (drill 0.8) (layers *.Cu *.Mask) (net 15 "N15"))
  (pad 6 thru_hole oval (at 7.62 5.08 90) (size 1.6 1.6) (drill 0.8) (layers *.Cu *.Mask) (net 8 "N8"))
  (pad 2 thru_hole oval (at 0 2.54 90) (size 1.6 1.6) (drill 0.8) (layers *.Cu *.Mask) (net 5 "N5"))
  (pad 5 thru_hole oval (at 7.62 7.62 90) (size 1.6 1.6) (drill 0.8) (layers *.Cu *.Mask))
  (pad 1 thru_hole rect (at 0 0 90) (size 1.6 1.6) (drill 0.8) (layers *.Cu *.Mask)))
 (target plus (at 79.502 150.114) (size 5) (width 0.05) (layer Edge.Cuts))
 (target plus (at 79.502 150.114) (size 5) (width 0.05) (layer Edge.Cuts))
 (gr_line (start 79.502 65.024) (end 79.502 120.396) (layer Edge.Cuts) (width 0.05))
 (gr_line (start 191.008 65.024) (end 79.502 65.024) (layer Edge.Cuts) (width 0.05))
 (gr_line (start 191.008 150.114) (end 191.008 65.024) (layer Edge.Cuts) (width 0.05))
 (gr_line (start 79.502 150.114) (end 191.008 150.114) (layer Edge.Cuts) (width 0.05))
 (gr_line (start 79.502 120.396) (end 79.502 150.114) (layer Edge.Cuts) (width 0.05))
 (segment (start 128.524 117.516872) (end 128.524 109.728) (width 0.25) (layer B.Cu) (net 6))
 (segment (start 128.524 109.728) (end 132.588 105.664) (width 0.25) (layer B.Cu) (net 6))
 (segment (start 132.588 105.664) (end 136.144 102.108) (width 0.25) (layer B.Cu) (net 6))
 (segment (start 136.144 102.108) (end 136.144 96.012) (width 0.25) (layer B.Cu) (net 6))
 (segment (start 136.144 96.012) (end 132.588 92.456) (width 0.25) (layer B.Cu) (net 6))
 (segment (start 132.588 91.948) (end 132.588 83.82) (width 0.25) (layer B.Cu) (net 6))
 (segment (start 132.588 92.456) (end 132.588 91.948) (width 0.25) (layer B.Cu) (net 6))
 (segment (start 91.186 119.888) (end 83.058 128.016) (width 0.5) (layer B.Cu) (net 6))
 (segment (start 128.524 117.516872) (end 126.152872 119.888) (width 0.5) (layer B.Cu) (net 6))
 (segment (start 126.152872 119.888) (end 91.186 119.888) (width 0.5) (layer B.Cu) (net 6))
 (segment (start 92.964 97.536) (end 92.964 101.6) (width 0.5) (layer F.Cu) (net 7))
 (segment (start 97.028 93.472) (end 92.964 97.536) (width 0.5) (layer F.Cu) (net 7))
 (segment (start 130.048 98.044) (end 125.476 93.472) (width 0.5) (layer F.Cu) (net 7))
 (segment (start 105.41 93.472) (end 104.284 93.472) (width 0.5) (layer F.Cu) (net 7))
 (segment (start 105.41 93.472) (end 97.028 93.472) (width 0.5) (layer F.Cu) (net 7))
 (segment (start 104.284 93.472) (end 100.584 97.172) (width 0.5) (layer F.Cu) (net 7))
 (segment (start 125.476 93.472) (end 105.41 93.472) (width 0.5) (layer F.Cu) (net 7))
 (segment (start 100.584 75.836) (end 104.03 72.39) (width 0.5) (layer F.Cu) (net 8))
 (segment (start 126.238 72.39) (end 130.048 76.2) (width 0.5) (layer F.Cu) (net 8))
 (segment (start 104.03 72.39) (end 126.238 72.39) (width 0.5) (layer F.Cu) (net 8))
 (segment (start 104.03 72.39) (end 97.79 72.39) (width 0.5) (layer F.Cu) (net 8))
 (segment (start 92.964 77.216) (end 92.964 80.772) (width 0.5) (layer F.Cu) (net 8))
 (segment (start 97.79 72.39) (end 92.964 77.216) (width 0.5) (layer F.Cu) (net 8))
 (segment (start 162.56 106.172) (end 160.02 108.712) (width 0.5) (layer F.Cu) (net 9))
 (segment (start 168.148 106.172) (end 162.56 106.172) (width 0.5) (layer F.Cu) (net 9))
 (segment (start 147.066 103.632) (end 141.224 109.474) (width 0.5) (layer F.Cu) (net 10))
 (segment (start 119.126 109.474) (end 115.824 106.172) (width 0.5) (layer F.Cu) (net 10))
 (segment (start 141.224 109.474) (end 119.126 109.474) (width 0.5) (layer F.Cu) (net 10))
 (segment (start 157.226 103.632) (end 158.242 103.632) (width 0.5) (layer F.Cu) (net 10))
 (segment (start 152.146 108.712) (end 157.226 103.632) (width 0.5) (layer F.Cu) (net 10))
 (segment (start 159.778001 101.841999) (end 157.988 103.632) (width 0.5) (layer F.Cu) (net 10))
 (segment (start 168.148 101.092) (end 167.398001 101.841999) (width 0.5) (layer F.Cu) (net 10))
 (segment (start 158.242 103.632) (end 157.988 103.632) (width 0.5) (layer F.Cu) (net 10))
 (segment (start 167.398001 101.841999) (end 159.778001 101.841999) (width 0.5) (layer F.Cu) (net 10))
 (segment (start 157.988 103.632) (end 147.066 103.632) (width 0.5) (layer F.Cu) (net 10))
 (segment (start 165.608 115.212002) (end 163.905001 116.915001) (width 0.5) (layer B.Cu) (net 3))
 (segment (start 165.608 103.632) (end 165.608 115.212002) (width 0.5) (layer B.Cu) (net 3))
 (segment (start 165.608 79.756) (end 169.672 79.756) (width 0.5) (layer F.Cu) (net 4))
 (segment (start 169.672 79.756) (end 170.942 81.026) (width 0.5) (layer F.Cu) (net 4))
 (segment (start 170.942 112.418002) (end 166.445001 116.915001) (width 0.5) (layer F.Cu) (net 4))
 (segment (start 170.942 81.026) (end 170.942 112.418002) (width 0.5) (layer F.Cu) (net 4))
 (segment (start 115.824 75.692) (end 119.126 78.994) (width 0.5) (layer F.Cu) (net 11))
 (segment (start 156.464 78.994) (end 155.702 78.994) (width 0.5) (layer F.Cu) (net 11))
 (segment (start 155.702 78.994) (end 152.4 75.692) (width 0.5) (layer F.Cu) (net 11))
 (segment (start 119.126 78.994) (end 156.464 78.994) (width 0.5) (layer F.Cu) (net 11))
 (segment (start 157.492001 77.965999) (end 156.464 78.994) (width 0.5) (layer F.Cu) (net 11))
 (segment (start 167.398001 77.965999) (end 157.492001 77.965999) (width 0.5) (layer F.Cu) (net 11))
 (segment (start 168.148 77.216) (end 167.398001 77.965999) (width 0.5) (layer F.Cu) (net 11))
 (segment (start 162.56 82.296) (end 168.148 82.296) (width 0.5) (layer F.Cu) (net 12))
 (segment (start 160.02 84.836) (end 162.56 82.296) (width 0.5) (layer F.Cu) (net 12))
 (segment (start 156.828 96.52) (end 160.02 99.712) (width 0.5) (layer B.Cu) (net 2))
 (segment (start 143.002 96.52) (end 156.828 96.52) (width 0.5) (layer B.Cu) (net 2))
 (segment (start 137.414 90.932) (end 143.002 96.52) (width 0.5) (layer B.Cu) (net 2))
 (segment (start 128.345001 68.655001) (end 137.414 77.724) (width 0.5) (layer B.Cu) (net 2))
 (segment (start 137.414 77.724) (end 137.414 90.932) (width 0.5) (layer B.Cu) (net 2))
 (segment (start 152.146 99.712) (end 147.176 99.712) (width 0.5) (layer F.Cu) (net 13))
 (segment (start 147.176 99.712) (end 139.192 107.696) (width 0.5) (layer F.Cu) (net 13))
 (segment (start 132.08 107.696) (end 130.048 105.664) (width 0.5) (layer F.Cu) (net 13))
 (segment (start 139.192 107.696) (end 132.08 107.696) (width 0.5) (layer F.Cu) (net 13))
 (segment (start 127.508 104.53263) (end 125.59137 102.616) (width 0.5) (layer F.Cu) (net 14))
 (segment (start 127.508 105.664) (end 127.508 104.53263) (width 0.5) (layer F.Cu) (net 14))
 (segment (start 112.124 102.616) (end 108.458 106.282) (width 0.5) (layer F.Cu) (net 14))
 (segment (start 104.14 102.616) (end 100.584 106.172) (width 0.5) (layer F.Cu) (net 14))
 (segment (start 112.522 102.616) (end 104.14 102.616) (width 0.5) (layer F.Cu) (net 14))
 (segment (start 112.522 102.616) (end 112.124 102.616) (width 0.5) (layer F.Cu) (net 14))
 (segment (start 125.59137 102.616) (end 112.522 102.616) (width 0.5) (layer F.Cu) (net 14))
 (segment (start 130.048 83.82) (end 132.842 86.614) (width 0.5) (layer F.Cu) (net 15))
 (segment (start 150.478 86.614) (end 152.4 84.692) (width 0.5) (layer F.Cu) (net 15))
 (segment (start 132.842 86.614) (end 150.478 86.614) (width 0.5) (layer F.Cu) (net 15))
 (segment (start 123.444 87.884) (end 127.508 83.82) (width 0.5) (layer F.Cu) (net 5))
 (segment (start 100.584 84.836) (end 103.632 87.884) (width 0.5) (layer F.Cu) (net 5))
 (segment (start 109.313999 85.691999) (end 111.506 87.884) (width 0.5) (layer F.Cu) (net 5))
 (segment (start 108.204 84.692) (end 109.203999 85.691999) (width 0.5) (layer F.Cu) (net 5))
 (segment (start 103.632 87.884) (end 111.506 87.884) (width 0.5) (layer F.Cu) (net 5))
 (segment (start 109.203999 85.691999) (end 109.313999 85.691999) (width 0.5) (layer F.Cu) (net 5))
 (segment (start 111.506 87.884) (end 123.444 87.884) (width 0.5) (layer F.Cu) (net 5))
 (segment (start 130.885001 68.655001) (end 134.112 71.882) (width 0.5) (layer F.Cu) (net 1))
 (segment (start 156.066 71.882) (end 160.02 75.836) (width 0.5) (layer F.Cu) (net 1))
 (segment (start 134.112 71.882) (end 156.066 71.882) (width 0.5) (layer F.Cu) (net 1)))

